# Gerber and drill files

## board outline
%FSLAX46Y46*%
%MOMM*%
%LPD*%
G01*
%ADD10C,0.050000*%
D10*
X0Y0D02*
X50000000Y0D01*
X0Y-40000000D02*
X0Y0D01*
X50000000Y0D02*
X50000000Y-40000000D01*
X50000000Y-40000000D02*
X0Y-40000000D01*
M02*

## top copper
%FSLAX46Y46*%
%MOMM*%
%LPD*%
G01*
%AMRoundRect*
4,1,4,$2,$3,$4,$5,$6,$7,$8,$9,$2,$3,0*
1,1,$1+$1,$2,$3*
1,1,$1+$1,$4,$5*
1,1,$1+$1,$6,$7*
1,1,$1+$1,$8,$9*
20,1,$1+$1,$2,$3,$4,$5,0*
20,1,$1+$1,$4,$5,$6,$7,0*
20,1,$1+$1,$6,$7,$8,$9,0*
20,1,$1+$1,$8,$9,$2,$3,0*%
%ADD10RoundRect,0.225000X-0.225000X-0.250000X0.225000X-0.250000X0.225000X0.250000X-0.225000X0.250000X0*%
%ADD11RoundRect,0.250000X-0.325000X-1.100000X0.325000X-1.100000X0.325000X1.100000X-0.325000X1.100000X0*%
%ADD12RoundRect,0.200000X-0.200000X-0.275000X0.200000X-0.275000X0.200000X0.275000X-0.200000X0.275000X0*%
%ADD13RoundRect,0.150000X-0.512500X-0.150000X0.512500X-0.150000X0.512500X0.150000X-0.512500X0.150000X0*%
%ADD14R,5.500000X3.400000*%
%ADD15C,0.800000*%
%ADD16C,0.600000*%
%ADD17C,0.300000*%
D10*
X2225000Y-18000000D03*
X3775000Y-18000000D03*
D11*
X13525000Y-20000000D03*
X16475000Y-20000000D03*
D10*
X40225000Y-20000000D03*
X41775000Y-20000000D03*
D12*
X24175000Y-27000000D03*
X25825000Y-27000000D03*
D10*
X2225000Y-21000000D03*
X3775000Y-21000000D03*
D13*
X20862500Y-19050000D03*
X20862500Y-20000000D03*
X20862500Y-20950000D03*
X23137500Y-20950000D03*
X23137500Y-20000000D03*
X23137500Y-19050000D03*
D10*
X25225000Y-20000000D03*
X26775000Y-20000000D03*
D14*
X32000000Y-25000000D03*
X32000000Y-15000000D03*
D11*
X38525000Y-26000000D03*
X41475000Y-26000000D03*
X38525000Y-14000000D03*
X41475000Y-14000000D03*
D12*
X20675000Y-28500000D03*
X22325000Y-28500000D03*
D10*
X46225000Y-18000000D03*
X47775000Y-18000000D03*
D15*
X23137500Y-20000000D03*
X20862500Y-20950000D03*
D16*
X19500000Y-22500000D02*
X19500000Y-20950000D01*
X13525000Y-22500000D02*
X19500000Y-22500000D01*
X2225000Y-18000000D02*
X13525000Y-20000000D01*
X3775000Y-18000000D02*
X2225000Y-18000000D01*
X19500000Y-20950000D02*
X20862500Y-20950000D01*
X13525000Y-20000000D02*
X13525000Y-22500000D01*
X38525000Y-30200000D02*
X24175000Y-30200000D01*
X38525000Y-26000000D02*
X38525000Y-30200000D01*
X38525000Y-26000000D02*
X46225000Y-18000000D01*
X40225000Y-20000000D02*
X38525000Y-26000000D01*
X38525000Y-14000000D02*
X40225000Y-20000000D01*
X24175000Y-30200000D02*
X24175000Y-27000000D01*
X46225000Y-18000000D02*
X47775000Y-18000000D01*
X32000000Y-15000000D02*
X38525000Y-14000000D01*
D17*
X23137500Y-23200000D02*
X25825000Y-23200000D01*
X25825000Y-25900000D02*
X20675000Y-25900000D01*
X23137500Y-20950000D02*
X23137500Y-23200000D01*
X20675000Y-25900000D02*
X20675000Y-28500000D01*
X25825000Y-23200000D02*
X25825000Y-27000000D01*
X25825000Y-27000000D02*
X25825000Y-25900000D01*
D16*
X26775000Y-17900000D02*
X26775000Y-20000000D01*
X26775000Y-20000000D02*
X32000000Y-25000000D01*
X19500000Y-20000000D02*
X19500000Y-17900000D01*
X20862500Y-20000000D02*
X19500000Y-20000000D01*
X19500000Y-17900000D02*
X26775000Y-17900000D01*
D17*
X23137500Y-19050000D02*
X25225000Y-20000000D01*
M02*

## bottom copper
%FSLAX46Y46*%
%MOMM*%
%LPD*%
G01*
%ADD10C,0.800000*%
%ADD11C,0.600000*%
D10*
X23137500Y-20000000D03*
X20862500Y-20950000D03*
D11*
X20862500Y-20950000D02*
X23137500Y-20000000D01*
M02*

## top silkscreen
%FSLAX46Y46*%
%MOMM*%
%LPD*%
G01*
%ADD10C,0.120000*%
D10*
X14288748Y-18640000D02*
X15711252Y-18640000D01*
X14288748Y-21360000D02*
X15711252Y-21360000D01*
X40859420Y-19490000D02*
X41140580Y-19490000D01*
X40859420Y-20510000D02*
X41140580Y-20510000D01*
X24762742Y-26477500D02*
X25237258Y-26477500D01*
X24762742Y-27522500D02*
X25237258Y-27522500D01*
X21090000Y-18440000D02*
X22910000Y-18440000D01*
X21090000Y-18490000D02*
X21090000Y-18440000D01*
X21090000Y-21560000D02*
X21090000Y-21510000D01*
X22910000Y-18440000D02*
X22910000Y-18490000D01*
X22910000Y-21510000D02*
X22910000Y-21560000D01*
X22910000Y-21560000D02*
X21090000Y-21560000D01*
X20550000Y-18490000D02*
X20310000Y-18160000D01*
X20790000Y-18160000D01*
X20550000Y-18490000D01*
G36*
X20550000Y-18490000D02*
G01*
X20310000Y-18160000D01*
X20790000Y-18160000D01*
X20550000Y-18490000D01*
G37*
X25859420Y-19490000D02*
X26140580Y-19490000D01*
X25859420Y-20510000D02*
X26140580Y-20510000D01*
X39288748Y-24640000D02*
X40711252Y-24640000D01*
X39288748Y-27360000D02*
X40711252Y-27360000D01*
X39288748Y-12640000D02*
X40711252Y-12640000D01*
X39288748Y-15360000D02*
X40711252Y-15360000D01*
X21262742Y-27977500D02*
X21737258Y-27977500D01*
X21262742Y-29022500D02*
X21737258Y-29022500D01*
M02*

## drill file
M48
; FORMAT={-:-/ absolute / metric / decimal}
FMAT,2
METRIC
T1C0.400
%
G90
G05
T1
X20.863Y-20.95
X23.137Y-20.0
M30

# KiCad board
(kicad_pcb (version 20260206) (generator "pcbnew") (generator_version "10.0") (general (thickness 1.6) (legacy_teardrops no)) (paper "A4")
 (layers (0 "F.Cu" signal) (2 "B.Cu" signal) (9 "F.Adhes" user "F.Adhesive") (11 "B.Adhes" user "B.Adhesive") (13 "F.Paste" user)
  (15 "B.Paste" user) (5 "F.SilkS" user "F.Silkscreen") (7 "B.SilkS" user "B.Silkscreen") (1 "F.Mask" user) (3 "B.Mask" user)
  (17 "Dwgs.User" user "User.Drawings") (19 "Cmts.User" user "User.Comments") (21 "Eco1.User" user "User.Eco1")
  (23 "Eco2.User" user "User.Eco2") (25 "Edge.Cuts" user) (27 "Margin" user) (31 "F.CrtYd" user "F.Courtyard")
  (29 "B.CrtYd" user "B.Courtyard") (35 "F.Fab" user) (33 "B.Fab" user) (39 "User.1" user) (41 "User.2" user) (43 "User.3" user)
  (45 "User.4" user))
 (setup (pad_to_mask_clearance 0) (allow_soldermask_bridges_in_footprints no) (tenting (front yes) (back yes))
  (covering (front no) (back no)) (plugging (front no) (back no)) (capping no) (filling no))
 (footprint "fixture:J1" (layer "F.Cu") (at 3 18)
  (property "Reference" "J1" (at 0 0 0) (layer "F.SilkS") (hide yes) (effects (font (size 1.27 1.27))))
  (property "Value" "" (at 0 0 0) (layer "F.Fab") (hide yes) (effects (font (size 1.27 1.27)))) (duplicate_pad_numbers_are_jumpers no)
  (pad "1" smd roundrect (at -0.775 0) (size 0.9 0.95) (layers "F.Cu" "F.Mask" "F.Paste") (roundrect_rratio 0.25) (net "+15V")
   (thermal_bridge_angle 45))
  (pad "2" smd roundrect (at 0.775 0) (size 0.9 0.95) (layers "F.Cu" "F.Mask" "F.Paste") (roundrect_rratio 0.25) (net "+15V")
   (thermal_bridge_angle 45)))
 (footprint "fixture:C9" (layer "F.Cu") (at 15 20)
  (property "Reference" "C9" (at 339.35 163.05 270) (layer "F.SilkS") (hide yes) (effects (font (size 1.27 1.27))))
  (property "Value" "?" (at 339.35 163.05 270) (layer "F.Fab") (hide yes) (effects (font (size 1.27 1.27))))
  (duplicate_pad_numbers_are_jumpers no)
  (fp_line (start -0.711252 -1.36) (end 0.711252 -1.36) (stroke (width 0.12) (type solid)) (layer "F.SilkS"))
  (fp_line (start -0.711252 1.36) (end 0.711252 1.36) (stroke (width 0.12) (type solid)) (layer "F.SilkS"))
  (pad "1" smd roundrect (at -1.475 0) (size 1.15 2.7) (layers "F.Cu" "F.Mask" "F.Paste") (roundrect_rratio 0.217391) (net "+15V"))
  (pad "2" smd roundrect (at 1.475 0) (size 1.15 2.7) (layers "F.Cu" "F.Mask" "F.Paste") (roundrect_rratio 0.217391) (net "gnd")))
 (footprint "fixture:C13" (layer "F.Cu") (at 41 20)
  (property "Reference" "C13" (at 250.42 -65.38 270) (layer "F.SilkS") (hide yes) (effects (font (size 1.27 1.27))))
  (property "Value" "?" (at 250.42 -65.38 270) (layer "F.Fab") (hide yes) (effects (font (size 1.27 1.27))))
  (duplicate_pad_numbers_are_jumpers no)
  (fp_line (start -0.14058 -0.51) (end 0.14058 -0.51) (stroke (width 0.12) (type solid)) (layer "F.SilkS"))
  (fp_line (start -0.14058 0.51) (end 0.14058 0.51) (stroke (width 0.12) (type solid)) (layer "F.SilkS"))
  (pad "1" smd roundrect (at -0.775 0) (size 0.9 0.95) (layers "F.Cu" "F.Mask" "F.Paste") (roundrect_rratio 0.25) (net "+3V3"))
  (pad "2" smd roundrect (at 0.775 0) (size 0.9 0.95) (layers "F.Cu" "F.Mask" "F.Paste") (roundrect_rratio 0.25) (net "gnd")))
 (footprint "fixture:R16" (layer "F.Cu") (at 25 27)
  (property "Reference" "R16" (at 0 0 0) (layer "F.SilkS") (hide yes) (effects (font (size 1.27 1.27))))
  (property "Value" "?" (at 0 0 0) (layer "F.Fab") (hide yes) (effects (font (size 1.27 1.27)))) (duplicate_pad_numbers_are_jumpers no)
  (fp_line (start -0.237258 -0.5225) (end 0.237258 -0.5225) (stroke (width 0.12) (type solid)) (layer "F.SilkS"))
  (fp_line (start -0.237258 0.5225) (end 0.237258 0.5225) (stroke (width 0.12) (type solid)) (layer "F.SilkS"))
  (pad "1" smd roundrect (at -0.825 0) (size 0.8 0.95) (layers "F.Cu" "F.Mask" "F.Paste") (roundrect_rratio 0.25) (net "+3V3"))
  (pad "2" smd roundrect (at 0.825 0) (size 0.8 0.95) (layers "F.Cu" "F.Mask" "F.Paste") (roundrect_rratio 0.25) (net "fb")))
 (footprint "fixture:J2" (layer "F.Cu") (at 3 21)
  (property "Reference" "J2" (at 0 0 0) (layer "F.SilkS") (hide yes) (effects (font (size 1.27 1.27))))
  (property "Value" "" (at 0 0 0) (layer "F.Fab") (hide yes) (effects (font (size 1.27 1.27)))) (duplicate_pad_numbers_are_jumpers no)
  (pad "1" smd roundrect (at -0.775 0) (size 0.9 0.95) (layers "F.Cu" "F.Mask" "F.Paste") (roundrect_rratio 0.25) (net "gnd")
   (thermal_bridge_angle 45))
  (pad "2" smd roundrect (at 0.775 0) (size 0.9 0.95) (layers "F.Cu" "F.Mask" "F.Paste") (roundrect_rratio 0.25) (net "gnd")
   (thermal_bridge_angle 45)))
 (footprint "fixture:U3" (layer "F.Cu") (at 22 20)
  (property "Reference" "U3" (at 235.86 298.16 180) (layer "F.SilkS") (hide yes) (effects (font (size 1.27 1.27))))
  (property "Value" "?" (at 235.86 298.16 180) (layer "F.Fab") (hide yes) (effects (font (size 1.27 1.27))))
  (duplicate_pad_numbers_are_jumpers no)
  (fp_line (start -0.91 -1.56) (end 0.91 -1.56) (stroke (width 0.12) (type solid)) (layer "F.SilkS"))
  (fp_line (start -0.91 -1.51) (end -0.91 -1.56) (stroke (width 0.12) (type solid)) (layer "F.SilkS"))
  (fp_line (start -0.91 1.56) (end -0.91 1.51) (stroke (width 0.12) (type solid)) (layer "F.SilkS"))
  (fp_line (start 0.91 -1.56) (end 0.91 -1.51) (stroke (width 0.12) (type solid)) (layer "F.SilkS"))
  (fp_line (start 0.91 1.51) (end 0.91 1.56) (stroke (width 0.12) (type solid)) (layer "F.SilkS"))
  (fp_line (start 0.91 1.56) (end -0.91 1.56) (stroke (width 0.12) (type solid)) (layer "F.SilkS"))
  (fp_poly (pts (xy -1.45 -1.51) (xy -1.69 -1.84) (xy -1.21 -1.84)) (stroke (width 0.12) (type solid)) (fill yes) (layer "F.SilkS"))
  (pad "1" smd roundrect (at -1.1375 -0.95) (size 1.325 0.6) (layers "F.Cu" "F.Mask" "F.Paste") (roundrect_rratio 0.25) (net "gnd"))
  (pad "2" smd roundrect (at -1.1375 0) (size 1.325 0.6) (layers "F.Cu" "F.Mask" "F.Paste") (roundrect_rratio 0.25) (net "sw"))
  (pad "3" smd roundrect (at -1.1375 0.95) (size 1.325 0.6) (layers "F.Cu" "F.Mask" "F.Paste") (roundrect_rratio 0.25) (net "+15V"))
  (pad "4" smd roundrect (at 1.1375 0.95) (size 1.325 0.6) (layers "F.Cu" "F.Mask" "F.Paste") (roundrect_rratio 0.25) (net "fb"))
  (pad "5" smd roundrect (at 1.1375 0) (size 1.325 0.6) (layers "F.Cu" "F.Mask" "F.Paste") (roundrect_rratio 0.25) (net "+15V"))
  (pad "6" smd roundrect (at 1.1375 -0.95) (size 1.325 0.6) (layers "F.Cu" "F.Mask" "F.Paste") (roundrect_rratio 0.25) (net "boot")))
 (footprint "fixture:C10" (layer "F.Cu") (at 26 20)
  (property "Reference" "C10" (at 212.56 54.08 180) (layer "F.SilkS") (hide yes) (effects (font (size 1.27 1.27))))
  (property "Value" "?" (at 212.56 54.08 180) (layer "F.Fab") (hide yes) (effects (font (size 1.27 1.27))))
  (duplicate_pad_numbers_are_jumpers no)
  (fp_line (start -0.14058 -0.51) (end 0.14058 -0.51) (stroke (width 0.12) (type solid)) (layer "F.SilkS"))
  (fp_line (start -0.14058 0.51) (end 0.14058 0.51) (stroke (width 0.12) (type solid)) (layer "F.SilkS"))
  (pad "1" smd roundrect (at -0.775 0) (size 0.9 0.95) (layers "F.Cu" "F.Mask" "F.Paste") (roundrect_rratio 0.25) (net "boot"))
  (pad "2" smd roundrect (at 0.775 0) (size 0.9 0.95) (layers "F.Cu" "F.Mask" "F.Paste") (roundrect_rratio 0.25) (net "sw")))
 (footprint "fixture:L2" (layer "F.Cu") (at 32 20 90)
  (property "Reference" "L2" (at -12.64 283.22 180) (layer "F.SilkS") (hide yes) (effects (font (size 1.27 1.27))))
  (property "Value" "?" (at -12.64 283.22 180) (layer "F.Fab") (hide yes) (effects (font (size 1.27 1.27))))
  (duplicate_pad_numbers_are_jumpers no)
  (pad "1" smd rect (at -5 0 90) (size 3.4 5.5) (layers "F.Cu" "F.Mask" "F.Paste") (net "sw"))
  (pad "2" smd rect (at 5 0 90) (size 3.4 5.5) (layers "F.Cu" "F.Mask" "F.Paste") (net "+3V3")))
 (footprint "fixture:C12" (layer "F.Cu") (at 40 26)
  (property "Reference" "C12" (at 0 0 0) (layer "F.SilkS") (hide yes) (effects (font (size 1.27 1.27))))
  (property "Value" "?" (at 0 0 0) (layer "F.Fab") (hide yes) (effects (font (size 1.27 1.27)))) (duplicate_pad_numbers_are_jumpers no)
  (fp_line (start -0.711252 -1.36) (end 0.711252 -1.36) (stroke (width 0.12) (type solid)) (layer "F.SilkS"))
  (fp_line (start -0.711252 1.36) (end 0.711252 1.36) (stroke (width 0.12) (type solid)) (layer "F.SilkS"))
  (pad "1" smd roundrect (at -1.475 0) (size 1.15 2.7) (layers "F.Cu" "F.Mask" "F.Paste") (roundrect_rratio 0.217391) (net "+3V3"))
  (pad "2" smd roundrect (at 1.475 0) (size 1.15 2.7) (layers "F.Cu" "F.Mask" "F.Paste") (roundrect_rratio 0.217391) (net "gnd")))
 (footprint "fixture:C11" (layer "F.Cu") (at 40 14)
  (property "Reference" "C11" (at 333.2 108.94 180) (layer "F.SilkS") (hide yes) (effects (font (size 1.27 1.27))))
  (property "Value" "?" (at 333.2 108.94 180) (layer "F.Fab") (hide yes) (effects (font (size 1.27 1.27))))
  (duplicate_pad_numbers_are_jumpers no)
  (fp_line (start -0.711252 -1.36) (end 0.711252 -1.36) (stroke (width 0.12) (type solid)) (layer "F.SilkS"))
  (fp_line (start -0.711252 1.36) (end 0.711252 1.36) (stroke (width 0.12) (type solid)) (layer "F.SilkS"))
  (pad "1" smd roundrect (at -1.475 0) (size 1.15 2.7) (layers "F.Cu" "F.Mask" "F.Paste") (roundrect_rratio 0.217391) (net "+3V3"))
  (pad "2" smd roundrect (at 1.475 0) (size 1.15 2.7) (layers "F.Cu" "F.Mask" "F.Paste") (roundrect_rratio 0.217391) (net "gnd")))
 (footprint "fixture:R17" (layer "F.Cu") (at 21.5 28.5)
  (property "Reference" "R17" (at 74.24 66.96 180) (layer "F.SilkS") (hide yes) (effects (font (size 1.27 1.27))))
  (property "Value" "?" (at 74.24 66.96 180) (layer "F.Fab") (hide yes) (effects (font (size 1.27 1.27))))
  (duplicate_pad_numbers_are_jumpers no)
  (fp_line (start -0.237258 -0.5225) (end 0.237258 -0.5225) (stroke (width 0.12) (type solid)) (layer "F.SilkS"))
  (fp_line (start -0.237258 0.5225) (end 0.237258 0.5225) (stroke (width 0.12) (type solid)) (layer "F.SilkS"))
  (pad "1" smd roundrect (at -0.825 0) (size 0.8 0.95) (layers "F.Cu" "F.Mask" "F.Paste") (roundrect_rratio 0.25) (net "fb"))
  (pad "2" smd roundrect (at 0.825 0) (size 0.8 0.95) (layers "F.Cu" "F.Mask" "F.Paste") (roundrect_rratio 0.25) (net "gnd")))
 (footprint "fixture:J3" (layer "F.Cu") (at 47 18)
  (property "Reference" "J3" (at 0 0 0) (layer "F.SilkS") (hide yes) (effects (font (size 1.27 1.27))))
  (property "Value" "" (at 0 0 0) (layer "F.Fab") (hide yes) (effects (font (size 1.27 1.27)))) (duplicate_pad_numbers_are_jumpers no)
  (pad "1" smd roundrect (at -0.775 0) (size 0.9 0.95) (layers "F.Cu" "F.Mask" "F.Paste") (roundrect_rratio 0.25) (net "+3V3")
   (thermal_bridge_angle 45))
  (pad "2" smd roundrect (at 0.775 0) (size 0.9 0.95) (layers "F.Cu" "F.Mask" "F.Paste") (roundrect_rratio 0.25) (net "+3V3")
   (thermal_bridge_angle 45)))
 (gr_line (start 0 0) (end 50 0) (stroke (width 0.05) (type default)) (layer "Edge.Cuts"))
 (gr_line (start 0 40) (end 0 0) (stroke (width 0.05) (type default)) (layer "Edge.Cuts"))
 (gr_line (start 50 0) (end 50 40) (stroke (width 0.05) (type default)) (layer "Edge.Cuts"))
 (gr_line (start 50 40) (end 0 40) (stroke (width 0.05) (type default)) (layer "Edge.Cuts"))
 (segment (start 19.5 22.5) (end 19.5 20.95) (width 0.6) (layer "F.Cu") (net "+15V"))
 (segment (start 13.525 22.5) (end 19.5 22.5) (width 0.6) (layer "F.Cu") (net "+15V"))
 (segment (start 2.225 18) (end 13.525 20) (width 0.6) (layer "F.Cu") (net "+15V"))
 (segment (start 3.775 18) (end 2.225 18) (width 0.6) (layer "F.Cu") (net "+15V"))
 (segment (start 19.5 20.95) (end 20.8625 20.95) (width 0.6) (layer "F.Cu") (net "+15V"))
 (segment (start 13.525 20) (end 13.525 22.5) (width 0.6) (layer "F.Cu") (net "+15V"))
 (via (at 23.1375 20) (size 0.8) (drill 0.4) (layers "F.Cu" "B.Cu") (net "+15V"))
 (via (at 20.8625 20.95) (size 0.8) (drill 0.4) (layers "F.Cu" "B.Cu") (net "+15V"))
 (segment (start 20.8625 20.95) (end 23.1375 20) (width 0.6) (layer "B.Cu") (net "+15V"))
 (segment (start 38.525 30.2) (end 24.175 30.2) (width 0.6) (layer "F.Cu") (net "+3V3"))
 (segment (start 38.525 26) (end 38.525 30.2) (width 0.6) (layer "F.Cu") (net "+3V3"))
 (segment (start 38.525 26) (end 46.225 18) (width 0.6) (layer "F.Cu") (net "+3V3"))
 (segment (start 40.225 20) (end 38.525 26) (width 0.6) (layer "F.Cu") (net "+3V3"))
 (segment (start 38.525 14) (end 40.225 20) (width 0.6) (layer "F.Cu") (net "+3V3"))
 (segment (start 24.175 30.2) (end 24.175 27) (width 0.6) (layer "F.Cu") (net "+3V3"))
 (segment (start 46.225 18) (end 47.775 18) (width 0.6) (layer "F.Cu") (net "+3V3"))
 (segment (start 32 15) (end 38.525 14) (width 0.6) (layer "F.Cu") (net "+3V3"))
 (segment (start 23.1375 23.2) (end 25.825 23.2) (width 0.3) (layer "F.Cu") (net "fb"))
 (segment (start 25.825 25.9) (end 20.675 25.9) (width 0.3) (layer "F.Cu") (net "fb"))
 (segment (start 23.1375 20.95) (end 23.1375 23.2) (width 0.3) (layer "F.Cu") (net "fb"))
 (segment (start 20.675 25.9) (end 20.675 28.5) (width 0.3) (layer "F.Cu") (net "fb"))
 (segment (start 25.825 23.2) (end 25.825 27) (width 0.3) (layer "F.Cu") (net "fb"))
 (segment (start 25.825 27) (end 25.825 25.9) (width 0.3) (layer "F.Cu") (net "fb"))
 (segment (start 26.775 17.9) (end 26.775 20) (width 0.6) (layer "F.Cu") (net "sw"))
 (segment (start 26.775 20) (end 32 25) (width 0.6) (layer "F.Cu") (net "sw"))
 (segment (start 19.5 20) (end 19.5 17.9) (width 0.6) (layer "F.Cu") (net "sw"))
 (segment (start 20.8625 20) (end 19.5 20) (width 0.6) (layer "F.Cu") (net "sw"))
 (segment (start 19.5 17.9) (end 26.775 17.9) (width 0.6) (layer "F.Cu") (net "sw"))
 (segment (start 23.1375 19.05) (end 25.225 20) (width 0.3) (layer "F.Cu") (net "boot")))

